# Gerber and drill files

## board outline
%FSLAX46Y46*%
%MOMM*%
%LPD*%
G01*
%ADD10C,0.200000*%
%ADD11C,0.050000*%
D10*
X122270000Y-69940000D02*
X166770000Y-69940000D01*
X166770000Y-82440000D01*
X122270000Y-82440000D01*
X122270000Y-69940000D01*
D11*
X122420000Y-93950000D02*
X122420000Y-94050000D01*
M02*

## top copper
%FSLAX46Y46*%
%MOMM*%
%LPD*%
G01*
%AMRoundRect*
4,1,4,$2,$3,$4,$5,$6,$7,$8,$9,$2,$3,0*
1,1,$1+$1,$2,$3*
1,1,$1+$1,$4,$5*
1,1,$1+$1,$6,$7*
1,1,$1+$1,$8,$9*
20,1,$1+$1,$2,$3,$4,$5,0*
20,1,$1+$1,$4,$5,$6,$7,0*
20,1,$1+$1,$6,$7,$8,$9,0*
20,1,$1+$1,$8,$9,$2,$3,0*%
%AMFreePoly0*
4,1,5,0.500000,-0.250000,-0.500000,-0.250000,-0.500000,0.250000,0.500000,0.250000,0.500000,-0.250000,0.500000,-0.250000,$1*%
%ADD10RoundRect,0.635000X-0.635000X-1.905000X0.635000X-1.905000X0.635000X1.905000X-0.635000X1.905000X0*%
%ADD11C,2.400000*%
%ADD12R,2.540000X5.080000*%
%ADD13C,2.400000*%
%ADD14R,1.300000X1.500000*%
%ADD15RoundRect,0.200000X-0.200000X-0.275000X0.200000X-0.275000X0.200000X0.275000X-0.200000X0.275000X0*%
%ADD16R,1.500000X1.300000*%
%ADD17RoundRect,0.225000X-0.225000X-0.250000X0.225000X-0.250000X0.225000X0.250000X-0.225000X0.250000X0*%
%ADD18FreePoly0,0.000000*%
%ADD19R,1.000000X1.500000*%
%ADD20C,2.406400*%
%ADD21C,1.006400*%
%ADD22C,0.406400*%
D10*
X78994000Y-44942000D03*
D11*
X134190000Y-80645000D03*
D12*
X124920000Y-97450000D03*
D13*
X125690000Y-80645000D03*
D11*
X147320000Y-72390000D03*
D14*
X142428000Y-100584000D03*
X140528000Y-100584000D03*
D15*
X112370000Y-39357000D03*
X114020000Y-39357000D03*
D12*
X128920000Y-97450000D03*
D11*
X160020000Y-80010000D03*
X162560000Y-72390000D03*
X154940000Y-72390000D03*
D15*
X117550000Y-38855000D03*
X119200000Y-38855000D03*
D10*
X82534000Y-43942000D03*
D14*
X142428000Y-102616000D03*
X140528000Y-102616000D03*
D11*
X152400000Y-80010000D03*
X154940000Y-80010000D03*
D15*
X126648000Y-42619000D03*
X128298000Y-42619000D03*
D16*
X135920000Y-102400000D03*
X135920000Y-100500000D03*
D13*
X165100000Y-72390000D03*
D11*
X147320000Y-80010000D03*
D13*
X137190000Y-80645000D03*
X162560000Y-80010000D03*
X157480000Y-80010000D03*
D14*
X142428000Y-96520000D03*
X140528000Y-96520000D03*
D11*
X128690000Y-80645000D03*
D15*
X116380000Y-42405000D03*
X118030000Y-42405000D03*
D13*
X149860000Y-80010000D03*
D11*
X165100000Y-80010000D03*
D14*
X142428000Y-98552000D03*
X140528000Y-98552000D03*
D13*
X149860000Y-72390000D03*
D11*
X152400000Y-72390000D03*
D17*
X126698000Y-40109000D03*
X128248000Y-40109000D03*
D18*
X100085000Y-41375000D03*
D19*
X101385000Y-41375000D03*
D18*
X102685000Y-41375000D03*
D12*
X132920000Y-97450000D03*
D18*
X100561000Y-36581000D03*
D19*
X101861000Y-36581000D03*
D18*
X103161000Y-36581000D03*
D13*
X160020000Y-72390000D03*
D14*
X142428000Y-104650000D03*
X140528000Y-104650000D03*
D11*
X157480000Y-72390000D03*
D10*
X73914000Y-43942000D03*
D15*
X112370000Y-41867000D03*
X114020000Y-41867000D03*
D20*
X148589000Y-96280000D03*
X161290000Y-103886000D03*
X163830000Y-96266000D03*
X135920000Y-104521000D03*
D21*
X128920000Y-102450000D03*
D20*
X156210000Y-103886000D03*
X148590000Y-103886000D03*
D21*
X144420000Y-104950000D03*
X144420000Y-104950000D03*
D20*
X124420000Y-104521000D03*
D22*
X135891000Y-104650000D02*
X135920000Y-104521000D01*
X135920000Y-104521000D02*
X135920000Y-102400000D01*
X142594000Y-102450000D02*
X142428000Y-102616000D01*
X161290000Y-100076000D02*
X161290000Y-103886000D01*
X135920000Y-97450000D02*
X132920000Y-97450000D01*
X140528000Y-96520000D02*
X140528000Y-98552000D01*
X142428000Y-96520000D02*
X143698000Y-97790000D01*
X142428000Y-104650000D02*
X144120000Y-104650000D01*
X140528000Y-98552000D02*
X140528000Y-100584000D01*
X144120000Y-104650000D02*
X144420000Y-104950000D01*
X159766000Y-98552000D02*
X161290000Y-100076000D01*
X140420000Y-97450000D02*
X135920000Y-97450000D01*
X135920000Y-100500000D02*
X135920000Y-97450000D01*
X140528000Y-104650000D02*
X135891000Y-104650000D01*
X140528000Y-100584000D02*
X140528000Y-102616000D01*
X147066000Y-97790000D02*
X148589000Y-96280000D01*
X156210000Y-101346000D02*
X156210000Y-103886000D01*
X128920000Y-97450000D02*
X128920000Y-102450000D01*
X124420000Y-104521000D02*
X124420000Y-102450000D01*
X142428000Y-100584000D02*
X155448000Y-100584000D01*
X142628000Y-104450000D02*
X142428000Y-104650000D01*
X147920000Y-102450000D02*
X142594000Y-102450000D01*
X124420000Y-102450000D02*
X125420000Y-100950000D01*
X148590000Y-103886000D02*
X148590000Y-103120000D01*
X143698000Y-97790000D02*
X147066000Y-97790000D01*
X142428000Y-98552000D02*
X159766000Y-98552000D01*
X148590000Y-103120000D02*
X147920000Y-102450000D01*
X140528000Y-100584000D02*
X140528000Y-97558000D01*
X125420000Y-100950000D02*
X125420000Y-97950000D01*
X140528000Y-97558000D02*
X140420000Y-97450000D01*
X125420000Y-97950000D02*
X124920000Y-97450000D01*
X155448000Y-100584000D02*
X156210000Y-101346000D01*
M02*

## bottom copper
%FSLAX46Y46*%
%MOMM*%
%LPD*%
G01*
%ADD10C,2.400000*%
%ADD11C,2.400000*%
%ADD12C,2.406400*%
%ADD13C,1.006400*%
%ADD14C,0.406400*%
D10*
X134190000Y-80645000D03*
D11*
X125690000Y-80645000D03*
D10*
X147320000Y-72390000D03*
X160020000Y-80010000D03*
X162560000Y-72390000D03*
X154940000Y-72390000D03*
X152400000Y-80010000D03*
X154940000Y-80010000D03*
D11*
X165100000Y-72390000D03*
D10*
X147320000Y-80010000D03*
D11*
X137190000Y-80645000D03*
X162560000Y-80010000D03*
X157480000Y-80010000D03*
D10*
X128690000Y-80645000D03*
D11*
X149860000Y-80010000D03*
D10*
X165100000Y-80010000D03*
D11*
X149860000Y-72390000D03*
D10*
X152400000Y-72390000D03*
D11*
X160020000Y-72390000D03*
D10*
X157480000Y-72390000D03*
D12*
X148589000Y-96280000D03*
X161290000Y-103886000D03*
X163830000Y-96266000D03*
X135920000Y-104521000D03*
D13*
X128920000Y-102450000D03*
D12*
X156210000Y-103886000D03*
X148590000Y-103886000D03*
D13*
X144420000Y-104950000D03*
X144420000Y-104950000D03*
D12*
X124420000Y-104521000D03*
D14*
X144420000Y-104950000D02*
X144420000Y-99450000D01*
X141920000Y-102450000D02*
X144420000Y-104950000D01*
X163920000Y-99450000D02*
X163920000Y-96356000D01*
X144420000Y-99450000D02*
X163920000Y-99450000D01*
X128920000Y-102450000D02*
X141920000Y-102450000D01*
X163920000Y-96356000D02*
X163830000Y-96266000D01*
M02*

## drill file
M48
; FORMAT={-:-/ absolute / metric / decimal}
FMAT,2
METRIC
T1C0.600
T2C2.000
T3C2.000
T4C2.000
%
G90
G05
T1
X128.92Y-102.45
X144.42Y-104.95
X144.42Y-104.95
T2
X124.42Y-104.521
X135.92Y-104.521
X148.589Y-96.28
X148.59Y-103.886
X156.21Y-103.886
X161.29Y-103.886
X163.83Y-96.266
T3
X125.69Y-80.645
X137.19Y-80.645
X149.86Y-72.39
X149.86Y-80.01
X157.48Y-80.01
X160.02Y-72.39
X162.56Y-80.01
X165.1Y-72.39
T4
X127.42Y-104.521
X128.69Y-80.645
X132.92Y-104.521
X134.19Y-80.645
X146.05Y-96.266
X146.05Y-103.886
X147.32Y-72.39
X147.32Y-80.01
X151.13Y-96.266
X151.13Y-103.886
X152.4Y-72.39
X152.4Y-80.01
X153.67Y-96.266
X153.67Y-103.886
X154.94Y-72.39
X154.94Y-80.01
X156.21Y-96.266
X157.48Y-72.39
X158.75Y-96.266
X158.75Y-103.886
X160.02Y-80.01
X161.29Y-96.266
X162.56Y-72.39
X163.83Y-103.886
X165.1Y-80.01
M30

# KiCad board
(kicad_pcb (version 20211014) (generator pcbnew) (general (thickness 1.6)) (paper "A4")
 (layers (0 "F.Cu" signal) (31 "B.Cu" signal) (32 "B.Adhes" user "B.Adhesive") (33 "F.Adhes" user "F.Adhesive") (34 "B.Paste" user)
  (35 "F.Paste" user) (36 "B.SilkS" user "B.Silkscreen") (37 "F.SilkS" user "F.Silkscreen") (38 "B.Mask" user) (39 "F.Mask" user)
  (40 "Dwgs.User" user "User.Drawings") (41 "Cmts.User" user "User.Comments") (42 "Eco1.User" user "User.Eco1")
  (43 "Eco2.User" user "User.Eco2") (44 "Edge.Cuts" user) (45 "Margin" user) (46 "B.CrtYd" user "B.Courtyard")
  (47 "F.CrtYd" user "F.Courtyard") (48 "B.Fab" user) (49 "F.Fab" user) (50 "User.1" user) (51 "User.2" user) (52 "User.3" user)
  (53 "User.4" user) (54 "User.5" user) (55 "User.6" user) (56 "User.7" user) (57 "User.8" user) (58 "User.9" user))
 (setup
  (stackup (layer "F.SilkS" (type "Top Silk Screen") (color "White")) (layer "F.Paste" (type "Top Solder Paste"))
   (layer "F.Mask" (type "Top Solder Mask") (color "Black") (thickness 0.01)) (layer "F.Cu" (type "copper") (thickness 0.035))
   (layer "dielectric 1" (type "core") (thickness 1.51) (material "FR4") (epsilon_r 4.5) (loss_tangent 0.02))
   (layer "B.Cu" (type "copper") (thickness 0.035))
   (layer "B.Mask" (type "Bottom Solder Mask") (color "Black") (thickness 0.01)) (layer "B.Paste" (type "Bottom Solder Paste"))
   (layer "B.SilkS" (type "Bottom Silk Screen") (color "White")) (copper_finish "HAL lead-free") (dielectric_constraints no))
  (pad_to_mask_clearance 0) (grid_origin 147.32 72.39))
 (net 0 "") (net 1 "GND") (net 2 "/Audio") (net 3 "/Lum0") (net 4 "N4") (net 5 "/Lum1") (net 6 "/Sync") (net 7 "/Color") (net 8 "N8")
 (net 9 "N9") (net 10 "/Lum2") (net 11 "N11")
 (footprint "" (layer "F.Cu") (at 153.67 103.886)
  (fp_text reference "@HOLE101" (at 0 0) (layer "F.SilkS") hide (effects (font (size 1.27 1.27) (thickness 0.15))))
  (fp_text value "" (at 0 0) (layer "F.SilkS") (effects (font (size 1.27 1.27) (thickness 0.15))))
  (pad "" np_thru_hole circle (at 0 0) (size 2 2) (drill 2) (layers *.Cu *.Mask)))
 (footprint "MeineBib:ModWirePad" (layer "F.Cu") (at 78.994 44.942)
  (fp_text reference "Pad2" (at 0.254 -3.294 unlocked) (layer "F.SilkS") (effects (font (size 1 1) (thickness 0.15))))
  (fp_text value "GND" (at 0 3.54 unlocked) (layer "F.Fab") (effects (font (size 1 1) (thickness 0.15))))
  (pad "1" smd roundrect (at 0 0) (size 2.54 5.08) (layers "F.Cu" "F.Paste" "F.Mask") (roundrect_rratio 0.25) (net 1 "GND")))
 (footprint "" (layer "F.Cu") (at 163.83 103.886)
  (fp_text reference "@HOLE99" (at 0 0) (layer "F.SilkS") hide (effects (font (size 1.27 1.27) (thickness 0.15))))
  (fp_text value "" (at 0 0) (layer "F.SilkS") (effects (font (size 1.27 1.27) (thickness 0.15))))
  (pad "" np_thru_hole circle (at 0 0) (size 2 2) (drill 2) (layers *.Cu *.Mask)))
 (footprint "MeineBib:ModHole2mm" (layer "F.Cu") (at 134.19 80.645)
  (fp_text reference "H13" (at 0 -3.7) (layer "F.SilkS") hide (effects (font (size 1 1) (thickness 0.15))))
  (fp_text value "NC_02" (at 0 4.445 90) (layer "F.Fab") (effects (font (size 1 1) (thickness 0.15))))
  (pad "" np_thru_hole circle (at 0 0) (size 2.4 2.4) (drill 2) (layers F&B.Cu *.Mask)))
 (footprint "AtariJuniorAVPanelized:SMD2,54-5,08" (layer "F.Cu") (at 124.92 97.45)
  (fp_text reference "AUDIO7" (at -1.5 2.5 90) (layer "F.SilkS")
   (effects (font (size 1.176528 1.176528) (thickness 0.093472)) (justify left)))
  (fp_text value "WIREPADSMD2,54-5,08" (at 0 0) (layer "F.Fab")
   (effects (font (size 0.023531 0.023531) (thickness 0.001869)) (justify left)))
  (pad "1" smd rect (at 0 0) (size 2.54 5.08) (layers "F.Cu" "F.Paste" "F.Mask") (solder_mask_margin 0.1016)))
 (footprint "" (layer "F.Cu") (at 151.13 96.266)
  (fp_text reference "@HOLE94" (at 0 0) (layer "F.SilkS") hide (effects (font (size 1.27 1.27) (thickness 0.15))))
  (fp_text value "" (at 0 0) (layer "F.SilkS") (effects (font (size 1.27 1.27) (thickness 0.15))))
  (pad "" np_thru_hole circle (at 0 0) (size 2 2) (drill 2) (layers *.Cu *.Mask)))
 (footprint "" (layer "F.Cu") (at 158.75 103.886)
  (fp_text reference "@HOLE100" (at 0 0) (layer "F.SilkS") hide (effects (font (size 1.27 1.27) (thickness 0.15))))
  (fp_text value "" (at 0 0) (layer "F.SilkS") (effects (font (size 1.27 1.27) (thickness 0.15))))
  (pad "" np_thru_hole circle (at 0 0) (size 2 2) (drill 2) (layers *.Cu *.Mask)))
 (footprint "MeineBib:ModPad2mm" (layer "F.Cu") (at 125.69 80.645)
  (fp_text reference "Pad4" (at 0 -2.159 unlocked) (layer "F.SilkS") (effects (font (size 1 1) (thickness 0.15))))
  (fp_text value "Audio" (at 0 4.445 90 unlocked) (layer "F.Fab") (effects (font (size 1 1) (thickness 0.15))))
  (pad "1" thru_hole circle (at 0 0) (size 2.4 2.4) (drill 2) (layers *.Cu *.Mask) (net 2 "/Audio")))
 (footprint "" (layer "F.Cu") (at 146.05 96.266)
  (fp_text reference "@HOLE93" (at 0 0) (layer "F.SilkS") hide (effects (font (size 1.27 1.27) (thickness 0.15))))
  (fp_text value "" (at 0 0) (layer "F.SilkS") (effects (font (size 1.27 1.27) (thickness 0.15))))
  (pad "" np_thru_hole circle (at 0 0) (size 2 2) (drill 2) (layers *.Cu *.Mask)))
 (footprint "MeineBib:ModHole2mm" (layer "F.Cu") (at 147.32 72.39)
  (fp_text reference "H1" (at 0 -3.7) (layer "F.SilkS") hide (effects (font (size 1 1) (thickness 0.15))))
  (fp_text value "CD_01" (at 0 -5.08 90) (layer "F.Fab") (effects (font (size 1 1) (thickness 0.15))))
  (pad "" np_thru_hole circle (at 0 0) (size 2.4 2.4) (drill 2) (layers F&B.Cu *.Mask)))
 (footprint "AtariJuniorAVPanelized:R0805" (layer "F.Cu") (at 141.478 100.584 180)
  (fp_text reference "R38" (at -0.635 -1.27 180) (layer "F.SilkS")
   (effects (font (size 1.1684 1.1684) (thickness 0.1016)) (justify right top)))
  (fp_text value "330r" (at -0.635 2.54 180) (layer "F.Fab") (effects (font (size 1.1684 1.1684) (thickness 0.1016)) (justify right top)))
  (pad "1" smd rect (at -0.95 0 180) (size 1.3 1.5) (layers "F.Cu" "F.Paste" "F.Mask") (solder_mask_margin 0.1016))
  (pad "2" smd rect (at 0.95 0 180) (size 1.3 1.5) (layers "F.Cu" "F.Paste" "F.Mask") (solder_mask_margin 0.1016)))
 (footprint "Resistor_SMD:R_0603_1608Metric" (layer "F.Cu") (at 113.195 39.357)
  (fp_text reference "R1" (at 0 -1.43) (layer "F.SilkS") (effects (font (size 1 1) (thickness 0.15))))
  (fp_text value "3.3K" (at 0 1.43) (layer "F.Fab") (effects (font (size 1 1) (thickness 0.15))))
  (pad "1" smd roundrect (at -0.825 0) (size 0.8 0.95) (layers "F.Cu" "F.Paste" "F.Mask") (roundrect_rratio 0.25) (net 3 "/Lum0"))
  (pad "2" smd roundrect (at 0.825 0) (size 0.8 0.95) (layers "F.Cu" "F.Paste" "F.Mask") (roundrect_rratio 0.25) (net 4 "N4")))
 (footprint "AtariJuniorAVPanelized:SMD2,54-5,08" (layer "F.Cu") (at 128.92 97.45)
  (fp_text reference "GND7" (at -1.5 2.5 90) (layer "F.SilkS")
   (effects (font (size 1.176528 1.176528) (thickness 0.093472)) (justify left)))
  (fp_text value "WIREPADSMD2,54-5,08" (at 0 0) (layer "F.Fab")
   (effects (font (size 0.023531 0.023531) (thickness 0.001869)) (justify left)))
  (pad "1" smd rect (at 0 0) (size 2.54 5.08) (layers "F.Cu" "F.Paste" "F.Mask") (solder_mask_margin 0.1016)))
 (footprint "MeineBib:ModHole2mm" (layer "F.Cu") (at 160.02 80.01 180)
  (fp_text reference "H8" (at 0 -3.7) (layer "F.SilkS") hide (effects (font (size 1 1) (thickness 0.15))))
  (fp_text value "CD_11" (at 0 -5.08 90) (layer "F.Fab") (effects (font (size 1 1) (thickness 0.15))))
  (pad "" np_thru_hole circle (at 0 0 180) (size 2.4 2.4) (drill 2) (layers F&B.Cu *.Mask)))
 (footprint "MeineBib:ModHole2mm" (layer "F.Cu") (at 162.56 72.39)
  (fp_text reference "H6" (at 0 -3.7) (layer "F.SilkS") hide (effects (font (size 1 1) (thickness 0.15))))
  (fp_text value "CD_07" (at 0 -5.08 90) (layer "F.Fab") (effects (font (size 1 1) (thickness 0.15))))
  (pad "" np_thru_hole circle (at 0 0) (size 2.4 2.4) (drill 2) (layers F&B.Cu *.Mask)))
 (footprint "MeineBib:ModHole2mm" (layer "F.Cu") (at 154.94 72.39)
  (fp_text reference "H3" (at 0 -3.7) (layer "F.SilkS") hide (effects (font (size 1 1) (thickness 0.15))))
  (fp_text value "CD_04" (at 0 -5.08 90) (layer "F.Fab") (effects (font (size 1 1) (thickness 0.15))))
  (pad "" np_thru_hole circle (at 0 0) (size 2.4 2.4) (drill 2) (layers F&B.Cu *.Mask)))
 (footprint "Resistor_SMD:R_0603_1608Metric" (layer "F.Cu") (at 118.375 38.855)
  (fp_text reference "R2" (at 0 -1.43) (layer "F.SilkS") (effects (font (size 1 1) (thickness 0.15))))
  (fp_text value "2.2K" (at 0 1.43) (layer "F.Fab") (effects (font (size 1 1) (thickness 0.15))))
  (pad "1" smd roundrect (at -0.825 0) (size 0.8 0.95) (layers "F.Cu" "F.Paste" "F.Mask") (roundrect_rratio 0.25) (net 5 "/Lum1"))
  (pad "2" smd roundrect (at 0.825 0) (size 0.8 0.95) (layers "F.Cu" "F.Paste" "F.Mask") (roundrect_rratio 0.25) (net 4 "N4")))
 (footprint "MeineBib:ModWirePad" (layer "F.Cu") (at 82.534 43.942)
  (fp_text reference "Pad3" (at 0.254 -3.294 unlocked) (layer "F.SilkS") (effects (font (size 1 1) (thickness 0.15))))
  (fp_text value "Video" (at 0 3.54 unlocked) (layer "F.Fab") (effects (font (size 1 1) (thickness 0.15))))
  (pad "1" smd roundrect (at 0 0) (size 2.54 5.08) (layers "F.Cu" "F.Paste" "F.Mask") (roundrect_rratio 0.25) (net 4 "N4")))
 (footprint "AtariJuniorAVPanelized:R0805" (layer "F.Cu") (at 141.478 102.616 180)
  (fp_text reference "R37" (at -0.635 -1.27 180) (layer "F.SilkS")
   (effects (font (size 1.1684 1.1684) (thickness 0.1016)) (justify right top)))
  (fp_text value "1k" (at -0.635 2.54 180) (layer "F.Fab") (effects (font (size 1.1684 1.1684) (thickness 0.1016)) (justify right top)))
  (pad "1" smd rect (at -0.95 0 180) (size 1.3 1.5) (layers "F.Cu" "F.Paste" "F.Mask") (solder_mask_margin 0.1016))
  (pad "2" smd rect (at 0.95 0 180) (size 1.3 1.5) (layers "F.Cu" "F.Paste" "F.Mask") (solder_mask_margin 0.1016)))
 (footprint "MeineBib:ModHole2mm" (layer "F.Cu") (at 152.4 80.01 180)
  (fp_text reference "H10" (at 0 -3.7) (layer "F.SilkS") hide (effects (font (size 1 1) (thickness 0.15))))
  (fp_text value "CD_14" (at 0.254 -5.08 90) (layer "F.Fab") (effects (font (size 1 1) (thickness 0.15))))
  (pad "" np_thru_hole circle (at 0 0 180) (size 2.4 2.4) (drill 2) (layers F&B.Cu *.Mask)))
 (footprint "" (layer "F.Cu") (at 153.67 96.266)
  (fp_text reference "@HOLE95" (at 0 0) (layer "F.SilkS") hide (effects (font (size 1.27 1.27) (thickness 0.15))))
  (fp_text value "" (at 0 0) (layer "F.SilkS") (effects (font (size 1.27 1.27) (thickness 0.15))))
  (pad "" np_thru_hole circle (at 0 0) (size 2 2) (drill 2) (layers *.Cu *.Mask)))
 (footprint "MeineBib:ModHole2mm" (layer "F.Cu") (at 154.94 80.01 180)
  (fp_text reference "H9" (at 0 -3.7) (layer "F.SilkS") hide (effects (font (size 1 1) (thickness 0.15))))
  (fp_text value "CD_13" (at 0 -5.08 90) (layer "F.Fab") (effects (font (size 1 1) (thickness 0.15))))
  (pad "" np_thru_hole circle (at 0 0 180) (size 2.4 2.4) (drill 2) (layers F&B.Cu *.Mask)))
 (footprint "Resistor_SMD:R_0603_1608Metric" (layer "F.Cu") (at 127.473 42.619)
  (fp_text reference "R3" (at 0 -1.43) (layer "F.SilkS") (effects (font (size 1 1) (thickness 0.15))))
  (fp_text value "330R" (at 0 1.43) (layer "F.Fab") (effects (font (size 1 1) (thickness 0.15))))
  (pad "1" smd roundrect (at -0.825 0) (size 0.8 0.95) (layers "F.Cu" "F.Paste" "F.Mask") (roundrect_rratio 0.25) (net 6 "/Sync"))
  (pad "2" smd roundrect (at 0.825 0) (size 0.8 0.95) (layers "F.Cu" "F.Paste" "F.Mask") (roundrect_rratio 0.25) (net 4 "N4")))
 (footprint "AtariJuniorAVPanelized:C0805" (layer "F.Cu") (at 135.92 101.45 90)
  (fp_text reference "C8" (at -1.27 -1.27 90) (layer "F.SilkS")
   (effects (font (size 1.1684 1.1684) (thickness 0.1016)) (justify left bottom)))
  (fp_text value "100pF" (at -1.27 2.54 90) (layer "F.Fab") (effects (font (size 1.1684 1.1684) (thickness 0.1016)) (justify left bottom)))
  (pad "1" smd rect (at -0.95 0 90) (size 1.3 1.5) (layers "F.Cu" "F.Paste" "F.Mask") (solder_mask_margin 0.1016))
  (pad "2" smd rect (at 0.95 0 90) (size 1.3 1.5) (layers "F.Cu" "F.Paste" "F.Mask") (solder_mask_margin 0.1016)))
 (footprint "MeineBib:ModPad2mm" (layer "F.Cu") (at 165.1 72.39)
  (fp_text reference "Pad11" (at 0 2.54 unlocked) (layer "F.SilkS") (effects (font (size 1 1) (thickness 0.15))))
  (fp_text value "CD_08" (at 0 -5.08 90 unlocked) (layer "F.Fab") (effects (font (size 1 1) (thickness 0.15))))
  (pad "1" thru_hole circle (at 0 0) (size 2.4 2.4) (drill 2) (layers *.Cu *.Mask) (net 1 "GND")))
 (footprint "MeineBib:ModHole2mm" (layer "F.Cu") (at 147.32 80.01 180)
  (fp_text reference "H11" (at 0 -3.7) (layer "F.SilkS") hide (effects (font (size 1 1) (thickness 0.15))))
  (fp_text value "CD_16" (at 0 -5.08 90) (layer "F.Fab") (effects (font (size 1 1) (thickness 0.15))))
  (pad "" np_thru_hole circle (at 0 0 180) (size 2.4 2.4) (drill 2) (layers F&B.Cu *.Mask)))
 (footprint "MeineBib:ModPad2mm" (layer "F.Cu") (at 137.19 80.645)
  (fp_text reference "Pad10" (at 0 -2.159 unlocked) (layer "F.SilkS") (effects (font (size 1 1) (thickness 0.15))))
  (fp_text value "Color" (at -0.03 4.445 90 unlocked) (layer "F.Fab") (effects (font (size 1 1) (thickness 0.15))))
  (pad "1" thru_hole circle (at 0 0) (size 2.4 2.4) (drill 2) (layers *.Cu *.Mask) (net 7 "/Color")))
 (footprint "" (layer "F.Cu") (at 146.05 103.886)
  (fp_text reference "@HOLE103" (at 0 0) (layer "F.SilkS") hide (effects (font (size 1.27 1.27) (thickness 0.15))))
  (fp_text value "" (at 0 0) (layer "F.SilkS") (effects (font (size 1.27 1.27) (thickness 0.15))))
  (pad "" np_thru_hole circle (at 0 0) (size 2 2) (drill 2) (layers *.Cu *.Mask)))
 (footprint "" (layer "F.Cu") (at 156.21 96.266)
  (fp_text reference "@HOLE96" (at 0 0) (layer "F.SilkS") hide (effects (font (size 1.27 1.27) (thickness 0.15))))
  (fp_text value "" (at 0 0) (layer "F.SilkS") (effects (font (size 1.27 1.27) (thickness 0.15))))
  (pad "" np_thru_hole circle (at 0 0) (size 2 2) (drill 2) (layers *.Cu *.Mask)))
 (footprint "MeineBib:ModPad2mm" (layer "F.Cu") (at 162.56 80.01)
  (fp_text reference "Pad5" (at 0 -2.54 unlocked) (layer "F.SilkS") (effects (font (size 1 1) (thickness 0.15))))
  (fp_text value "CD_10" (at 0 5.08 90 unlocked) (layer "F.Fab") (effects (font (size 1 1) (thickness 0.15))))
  (pad "1" thru_hole circle (at 0 0) (size 2.4 2.4) (drill 2) (layers *.Cu *.Mask) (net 5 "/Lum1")))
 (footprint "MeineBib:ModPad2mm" (layer "F.Cu") (at 157.48 80.01)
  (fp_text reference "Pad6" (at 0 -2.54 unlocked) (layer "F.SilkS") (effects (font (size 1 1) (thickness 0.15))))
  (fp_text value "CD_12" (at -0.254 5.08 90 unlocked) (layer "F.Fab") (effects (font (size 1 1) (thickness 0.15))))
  (pad "1" thru_hole circle (at 0 0) (size 2.4 2.4) (drill 2) (layers *.Cu *.Mask) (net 6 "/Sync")))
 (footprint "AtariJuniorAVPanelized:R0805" (layer "F.Cu") (at 141.478 96.52 180)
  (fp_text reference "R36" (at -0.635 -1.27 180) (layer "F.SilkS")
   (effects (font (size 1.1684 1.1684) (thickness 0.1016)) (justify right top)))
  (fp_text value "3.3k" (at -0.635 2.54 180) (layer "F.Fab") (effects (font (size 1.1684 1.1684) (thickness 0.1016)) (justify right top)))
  (pad "1" smd rect (at -0.95 0 180) (size 1.3 1.5) (layers "F.Cu" "F.Paste" "F.Mask") (solder_mask_margin 0.1016))
  (pad "2" smd rect (at 0.95 0 180) (size 1.3 1.5) (layers "F.Cu" "F.Paste" "F.Mask") (solder_mask_margin 0.1016)))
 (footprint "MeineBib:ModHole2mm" (layer "F.Cu") (at 128.69 80.645)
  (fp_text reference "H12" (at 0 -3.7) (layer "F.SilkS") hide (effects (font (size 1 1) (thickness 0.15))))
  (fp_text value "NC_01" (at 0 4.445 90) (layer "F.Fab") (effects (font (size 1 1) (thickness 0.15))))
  (pad "" np_thru_hole circle (at 0 0) (size 2.4 2.4) (drill 2) (layers F&B.Cu *.Mask)))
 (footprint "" (layer "F.Cu") (at 127.42 104.521)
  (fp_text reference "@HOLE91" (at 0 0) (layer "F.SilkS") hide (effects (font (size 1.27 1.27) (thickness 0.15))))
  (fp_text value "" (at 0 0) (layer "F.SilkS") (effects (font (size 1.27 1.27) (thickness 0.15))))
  (pad "" np_thru_hole circle (at 0 0) (size 2 2) (drill 2) (layers *.Cu *.Mask)))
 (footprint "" (layer "F.Cu") (at 161.29 96.266)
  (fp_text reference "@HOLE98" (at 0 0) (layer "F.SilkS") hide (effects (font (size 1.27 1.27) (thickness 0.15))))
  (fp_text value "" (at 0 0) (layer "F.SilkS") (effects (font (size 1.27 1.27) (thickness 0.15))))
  (pad "" np_thru_hole circle (at 0 0) (size 2 2) (drill 2) (layers *.Cu *.Mask)))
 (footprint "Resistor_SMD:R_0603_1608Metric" (layer "F.Cu") (at 117.205 42.405)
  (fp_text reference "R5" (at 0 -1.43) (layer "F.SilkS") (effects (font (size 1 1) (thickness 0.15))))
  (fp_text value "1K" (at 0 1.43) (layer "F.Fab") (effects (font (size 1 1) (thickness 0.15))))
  (pad "1" smd roundrect (at -0.825 0) (size 0.8 0.95) (layers "F.Cu" "F.Paste" "F.Mask") (roundrect_rratio 0.25) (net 1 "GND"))
  (pad "2" smd roundrect (at 0.825 0) (size 0.8 0.95) (layers "F.Cu" "F.Paste" "F.Mask") (roundrect_rratio 0.25) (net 7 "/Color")))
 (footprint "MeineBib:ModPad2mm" (layer "F.Cu") (at 149.86 80.01)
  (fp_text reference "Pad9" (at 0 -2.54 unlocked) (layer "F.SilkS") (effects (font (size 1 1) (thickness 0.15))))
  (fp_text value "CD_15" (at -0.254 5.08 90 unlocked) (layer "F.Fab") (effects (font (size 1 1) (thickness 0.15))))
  (pad "1" thru_hole circle (at 0 0) (size 2.4 2.4) (drill 2) (layers *.Cu *.Mask) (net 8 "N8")))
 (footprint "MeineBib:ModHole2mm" (layer "F.Cu") (at 165.1 80.01 180)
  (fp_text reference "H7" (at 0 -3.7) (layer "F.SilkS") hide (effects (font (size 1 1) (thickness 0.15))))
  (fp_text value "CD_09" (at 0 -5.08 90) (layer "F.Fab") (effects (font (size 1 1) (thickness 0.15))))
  (pad "" np_thru_hole circle (at 0 0 180) (size 2.4 2.4) (drill 2) (layers F&B.Cu *.Mask)))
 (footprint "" (layer "F.Cu") (at 158.75 96.266)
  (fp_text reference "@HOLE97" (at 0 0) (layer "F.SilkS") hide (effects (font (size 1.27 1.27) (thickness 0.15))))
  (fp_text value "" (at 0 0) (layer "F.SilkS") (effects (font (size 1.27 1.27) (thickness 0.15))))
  (pad "" np_thru_hole circle (at 0 0) (size 2 2) (drill 2) (layers *.Cu *.Mask)))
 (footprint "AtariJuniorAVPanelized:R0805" (layer "F.Cu") (at 141.478 98.552 180)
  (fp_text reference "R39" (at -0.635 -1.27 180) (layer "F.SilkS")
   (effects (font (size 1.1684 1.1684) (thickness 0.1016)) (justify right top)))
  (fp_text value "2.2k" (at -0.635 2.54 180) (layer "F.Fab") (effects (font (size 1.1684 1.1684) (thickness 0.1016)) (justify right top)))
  (pad "1" smd rect (at -0.95 0 180) (size 1.3 1.5) (layers "F.Cu" "F.Paste" "F.Mask") (solder_mask_margin 0.1016))
  (pad "2" smd rect (at 0.95 0 180) (size 1.3 1.5) (layers "F.Cu" "F.Paste" "F.Mask") (solder_mask_margin 0.1016)))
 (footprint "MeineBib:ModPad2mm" (layer "F.Cu") (at 149.86 72.39)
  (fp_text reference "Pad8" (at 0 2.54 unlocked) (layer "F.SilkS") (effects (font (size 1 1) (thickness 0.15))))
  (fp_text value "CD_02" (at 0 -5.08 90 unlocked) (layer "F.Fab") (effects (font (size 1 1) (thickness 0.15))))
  (pad "1" thru_hole circle (at 0 0) (size 2.4 2.4) (drill 2) (layers *.Cu *.Mask) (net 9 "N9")))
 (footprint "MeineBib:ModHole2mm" (layer "F.Cu") (at 152.4 72.39)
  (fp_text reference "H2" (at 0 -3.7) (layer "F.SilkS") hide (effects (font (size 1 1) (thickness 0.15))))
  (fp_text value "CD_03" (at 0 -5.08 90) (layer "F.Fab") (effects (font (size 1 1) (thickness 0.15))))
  (pad "" np_thru_hole circle (at 0 0) (size 2.4 2.4) (drill 2) (layers F&B.Cu *.Mask)))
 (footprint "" (layer "F.Cu") (at 132.92 104.521)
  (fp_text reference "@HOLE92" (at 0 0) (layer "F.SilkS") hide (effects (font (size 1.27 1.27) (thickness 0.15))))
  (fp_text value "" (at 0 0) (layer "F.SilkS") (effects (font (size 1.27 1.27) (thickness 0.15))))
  (pad "" np_thru_hole circle (at 0 0) (size 2 2) (drill 2) (layers *.Cu *.Mask)))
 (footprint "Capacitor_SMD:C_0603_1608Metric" (layer "F.Cu") (at 127.473 40.109)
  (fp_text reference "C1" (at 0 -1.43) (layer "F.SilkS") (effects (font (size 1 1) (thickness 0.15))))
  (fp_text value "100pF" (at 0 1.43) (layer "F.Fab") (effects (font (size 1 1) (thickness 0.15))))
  (pad "1" smd roundrect (at -0.775 0) (size 0.9 0.95) (layers "F.Cu" "F.Paste" "F.Mask") (roundrect_rratio 0.25) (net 4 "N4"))
  (pad "2" smd roundrect (at 0.775 0) (size 0.9 0.95) (layers "F.Cu" "F.Paste" "F.Mask") (roundrect_rratio 0.25) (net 7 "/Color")))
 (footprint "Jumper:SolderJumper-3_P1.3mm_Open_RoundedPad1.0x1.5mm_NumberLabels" (layer "F.Cu") (at 101.385 41.375)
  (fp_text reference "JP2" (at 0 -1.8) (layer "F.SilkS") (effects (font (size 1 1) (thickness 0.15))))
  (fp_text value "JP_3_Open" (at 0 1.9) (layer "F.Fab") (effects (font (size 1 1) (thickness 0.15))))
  (pad "1" smd custom (at -1.3 0) (size 1 0.5) (layers "F.Cu" "F.Mask") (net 8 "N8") (zone_connect 2)
   (options (clearance outline) (anchor rect)) (primitives))
  (pad "2" smd rect (at 0 0) (size 1 1.5) (layers "F.Cu" "F.Mask") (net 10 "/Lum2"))
  (pad "3" smd custom (at 1.3 0) (size 1 0.5) (layers "F.Cu" "F.Mask") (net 9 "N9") (zone_connect 2)
   (options (clearance outline) (anchor rect)) (primitives)))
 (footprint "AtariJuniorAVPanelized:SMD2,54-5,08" (layer "F.Cu") (at 132.92 97.45)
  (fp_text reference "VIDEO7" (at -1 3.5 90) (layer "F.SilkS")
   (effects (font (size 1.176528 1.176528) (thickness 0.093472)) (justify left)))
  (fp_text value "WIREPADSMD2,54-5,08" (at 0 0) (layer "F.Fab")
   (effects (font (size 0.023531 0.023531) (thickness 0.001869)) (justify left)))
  (pad "1" smd rect (at 0 0) (size 2.54 5.08) (layers "F.Cu" "F.Paste" "F.Mask") (solder_mask_margin 0.1016)))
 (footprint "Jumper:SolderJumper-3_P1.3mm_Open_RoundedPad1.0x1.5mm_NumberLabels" (layer "F.Cu") (at 101.861 36.581)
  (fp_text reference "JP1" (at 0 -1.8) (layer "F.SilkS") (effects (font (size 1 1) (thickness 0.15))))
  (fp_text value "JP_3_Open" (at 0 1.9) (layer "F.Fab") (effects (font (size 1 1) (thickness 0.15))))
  (pad "1" smd custom (at -1.3 0) (size 1 0.5) (layers "F.Cu" "F.Mask") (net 9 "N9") (zone_connect 2)
   (options (clearance outline) (anchor rect)) (primitives))
  (pad "2" smd rect (at 0 0) (size 1 1.5) (layers "F.Cu" "F.Mask") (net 3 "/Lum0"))
  (pad "3" smd custom (at 1.3 0) (size 1 0.5) (layers "F.Cu" "F.Mask") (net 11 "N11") (zone_connect 2)
   (options (clearance outline) (anchor rect)) (primitives)))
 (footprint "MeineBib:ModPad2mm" (layer "F.Cu") (at 160.02 72.39)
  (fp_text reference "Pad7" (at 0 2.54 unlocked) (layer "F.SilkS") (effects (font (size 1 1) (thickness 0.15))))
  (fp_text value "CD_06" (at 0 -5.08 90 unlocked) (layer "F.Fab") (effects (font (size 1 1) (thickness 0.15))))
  (pad "1" thru_hole circle (at 0 0) (size 2.4 2.4) (drill 2) (layers *.Cu *.Mask) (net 11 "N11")))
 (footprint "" (layer "F.Cu") (at 151.13 103.886)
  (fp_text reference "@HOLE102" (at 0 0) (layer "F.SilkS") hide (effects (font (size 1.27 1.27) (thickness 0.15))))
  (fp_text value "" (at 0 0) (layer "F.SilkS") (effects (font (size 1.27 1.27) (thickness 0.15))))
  (pad "" np_thru_hole circle (at 0 0) (size 2 2) (drill 2) (layers *.Cu *.Mask)))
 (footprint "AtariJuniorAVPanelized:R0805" (layer "F.Cu") (at 141.478 104.65 180)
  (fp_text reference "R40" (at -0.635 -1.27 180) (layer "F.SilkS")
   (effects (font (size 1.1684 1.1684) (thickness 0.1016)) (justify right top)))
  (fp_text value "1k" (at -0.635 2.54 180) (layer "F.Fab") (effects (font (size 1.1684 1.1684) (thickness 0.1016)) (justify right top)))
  (pad "1" smd rect (at -0.95 0 180) (size 1.3 1.5) (layers "F.Cu" "F.Paste" "F.Mask") (solder_mask_margin 0.1016))
  (pad "2" smd rect (at 0.95 0 180) (size 1.3 1.5) (layers "F.Cu" "F.Paste" "F.Mask") (solder_mask_margin 0.1016)))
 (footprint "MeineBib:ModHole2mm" (layer "F.Cu") (at 157.48 72.39)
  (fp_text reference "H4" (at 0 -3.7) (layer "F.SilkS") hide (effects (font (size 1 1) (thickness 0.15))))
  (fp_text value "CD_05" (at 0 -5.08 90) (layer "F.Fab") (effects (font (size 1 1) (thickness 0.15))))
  (pad "" np_thru_hole circle (at 0 0) (size 2.4 2.4) (drill 2) (layers F&B.Cu *.Mask)))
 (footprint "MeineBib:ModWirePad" (layer "F.Cu") (at 73.914 43.942)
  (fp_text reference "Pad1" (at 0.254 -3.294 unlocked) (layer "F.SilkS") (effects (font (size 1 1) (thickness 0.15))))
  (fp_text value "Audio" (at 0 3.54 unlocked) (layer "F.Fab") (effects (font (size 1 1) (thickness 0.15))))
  (pad "1" smd roundrect (at 0 0) (size 2.54 5.08) (layers "F.Cu" "F.Paste" "F.Mask") (roundrect_rratio 0.25) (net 2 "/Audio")))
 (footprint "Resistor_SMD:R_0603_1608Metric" (layer "F.Cu") (at 113.195 41.867)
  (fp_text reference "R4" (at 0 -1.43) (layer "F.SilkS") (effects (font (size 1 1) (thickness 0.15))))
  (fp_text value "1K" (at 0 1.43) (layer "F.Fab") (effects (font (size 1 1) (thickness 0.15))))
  (pad "1" smd roundrect (at -0.825 0) (size 0.8 0.95) (layers "F.Cu" "F.Paste" "F.Mask") (roundrect_rratio 0.25) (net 10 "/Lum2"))
  (pad "2" smd roundrect (at 0.825 0) (size 0.8 0.95) (layers "F.Cu" "F.Paste" "F.Mask") (roundrect_rratio 0.25) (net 4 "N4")))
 (gr_rect (start 122.27 82.44) (end 166.77 69.94) (layer "Edge.Cuts") (width 0.2) (fill none))
 (gr_line (start 122.42 93.95) (end 122.42 94.05) (layer "Edge.Cuts") (width 0.05))
 (segment (start 135.891 104.65) (end 135.92 104.521) (width 0.4064) (layer "F.Cu") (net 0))
 (segment (start 135.92 104.521) (end 135.92 102.4) (width 0.4064) (layer "F.Cu") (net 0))
 (segment (start 142.594 102.45) (end 142.428 102.616) (width 0.4064) (layer "F.Cu") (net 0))
 (segment (start 161.29 100.076) (end 161.29 103.886) (width 0.4064) (layer "F.Cu") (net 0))
 (segment (start 135.92 97.45) (end 132.92 97.45) (width 0.4064) (layer "F.Cu") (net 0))
 (segment (start 140.528 96.52) (end 140.528 98.552) (width 0.4064) (layer "F.Cu") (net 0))
 (segment (start 142.428 96.52) (end 143.698 97.79) (width 0.4064) (layer "F.Cu") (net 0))
 (segment (start 142.428 104.65) (end 144.12 104.65) (width 0.4064) (layer "F.Cu") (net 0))
 (segment (start 140.528 98.552) (end 140.528 100.584) (width 0.4064) (layer "F.Cu") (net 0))
 (segment (start 144.12 104.65) (end 144.42 104.95) (width 0.4064) (layer "F.Cu") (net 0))
 (segment (start 159.766 98.552) (end 161.29 100.076) (width 0.4064) (layer "F.Cu") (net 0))
 (segment (start 140.42 97.45) (end 135.92 97.45) (width 0.4064) (layer "F.Cu") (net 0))
 (segment (start 135.92 100.5) (end 135.92 97.45) (width 0.4064) (layer "F.Cu") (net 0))
 (segment (start 140.528 104.65) (end 135.891 104.65) (width 0.4064) (layer "F.Cu") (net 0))
 (segment (start 140.528 100.584) (end 140.528 102.616) (width 0.4064) (layer "F.Cu") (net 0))
 (segment (start 147.066 97.79) (end 148.589 96.28) (width 0.4064) (layer "F.Cu") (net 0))
 (segment (start 156.21 101.346) (end 156.21 103.886) (width 0.4064) (layer "F.Cu") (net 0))
 (segment (start 128.92 97.45) (end 128.92 102.45) (width 0.4064) (layer "F.Cu") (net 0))
 (segment (start 124.42 104.521) (end 124.42 102.45) (width 0.4064) (layer "F.Cu") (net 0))
 (segment (start 142.428 100.584) (end 155.448 100.584) (width 0.4064) (layer "F.Cu") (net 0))
 (segment (start 142.628 104.45) (end 142.428 104.65) (width 0.4064) (layer "F.Cu") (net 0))
 (segment (start 147.92 102.45) (end 142.594 102.45) (width 0.4064) (layer "F.Cu") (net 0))
 (segment (start 124.42 102.45) (end 125.42 100.95) (width 0.4064) (layer "F.Cu") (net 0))
 (segment (start 148.59 103.886) (end 148.59 103.12) (width 0.4064) (layer "F.Cu") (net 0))
 (segment (start 143.698 97.79) (end 147.066 97.79) (width 0.4064) (layer "F.Cu") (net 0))
 (segment (start 142.428 98.552) (end 159.766 98.552) (width 0.4064) (layer "F.Cu") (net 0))
 (segment (start 148.59 103.12) (end 147.92 102.45) (width 0.4064) (layer "F.Cu") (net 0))
 (segment (start 140.528 100.584) (end 140.528 97.558) (width 0.4064) (layer "F.Cu") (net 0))
 (segment (start 125.42 100.95) (end 125.42 97.95) (width 0.4064) (layer "F.Cu") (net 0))
 (segment (start 140.528 97.558) (end 140.42 97.45) (width 0.4064) (layer "F.Cu") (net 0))
 (segment (start 125.42 97.95) (end 124.92 97.45) (width 0.4064) (layer "F.Cu") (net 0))
 (segment (start 155.448 100.584) (end 156.21 101.346) (width 0.4064) (layer "F.Cu") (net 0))
 (via (at 148.589 96.28) (size 2.4064) (drill 2) (layers "F.Cu" "B.Cu") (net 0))
 (via (at 161.29 103.886) (size 2.4064) (drill 2) (layers "F.Cu" "B.Cu") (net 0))
 (via (at 163.83 96.266) (size 2.4064) (drill 2) (layers "F.Cu" "B.Cu") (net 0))
 (via (at 135.92 104.521) (size 2.4064) (drill 2) (layers "F.Cu" "B.Cu") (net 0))
 (via (at 128.92 102.45) (size 1.0064) (drill 0.6) (layers "F.Cu" "B.Cu") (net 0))
 (via (at 156.21 103.886) (size 2.4064) (drill 2) (layers "F.Cu" "B.Cu") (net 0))
 (via (at 148.59 103.886) (size 2.4064) (drill 2) (layers "F.Cu" "B.Cu") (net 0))
 (via (at 144.42 104.95) (size 1.0064) (drill 0.6) (layers "F.Cu" "B.Cu") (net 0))
 (via (at 144.42 104.95) (size 1.0064) (drill 0.6) (layers "F.Cu" "B.Cu") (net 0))
 (via (at 124.42 104.521) (size 2.4064) (drill 2) (layers "F.Cu" "B.Cu") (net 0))
 (segment (start 144.42 104.95) (end 144.42 99.45) (width 0.4064) (layer "B.Cu") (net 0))
 (segment (start 141.92 102.45) (end 144.42 104.95) (width 0.4064) (layer "B.Cu") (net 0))
 (segment (start 163.92 99.45) (end 163.92 96.356) (width 0.4064) (layer "B.Cu") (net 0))
 (segment (start 144.42 99.45) (end 163.92 99.45) (width 0.4064) (layer "B.Cu") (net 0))
 (segment (start 128.92 102.45) (end 141.92 102.45) (width 0.4064) (layer "B.Cu") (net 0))
 (segment (start 163.92 96.356) (end 163.83 96.266) (width 0.4064) (layer "B.Cu") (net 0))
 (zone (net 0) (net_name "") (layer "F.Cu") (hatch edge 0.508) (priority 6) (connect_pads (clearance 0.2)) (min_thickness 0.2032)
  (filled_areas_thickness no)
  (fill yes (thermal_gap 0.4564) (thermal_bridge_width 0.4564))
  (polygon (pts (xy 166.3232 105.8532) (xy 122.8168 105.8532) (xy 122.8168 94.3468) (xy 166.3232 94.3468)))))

